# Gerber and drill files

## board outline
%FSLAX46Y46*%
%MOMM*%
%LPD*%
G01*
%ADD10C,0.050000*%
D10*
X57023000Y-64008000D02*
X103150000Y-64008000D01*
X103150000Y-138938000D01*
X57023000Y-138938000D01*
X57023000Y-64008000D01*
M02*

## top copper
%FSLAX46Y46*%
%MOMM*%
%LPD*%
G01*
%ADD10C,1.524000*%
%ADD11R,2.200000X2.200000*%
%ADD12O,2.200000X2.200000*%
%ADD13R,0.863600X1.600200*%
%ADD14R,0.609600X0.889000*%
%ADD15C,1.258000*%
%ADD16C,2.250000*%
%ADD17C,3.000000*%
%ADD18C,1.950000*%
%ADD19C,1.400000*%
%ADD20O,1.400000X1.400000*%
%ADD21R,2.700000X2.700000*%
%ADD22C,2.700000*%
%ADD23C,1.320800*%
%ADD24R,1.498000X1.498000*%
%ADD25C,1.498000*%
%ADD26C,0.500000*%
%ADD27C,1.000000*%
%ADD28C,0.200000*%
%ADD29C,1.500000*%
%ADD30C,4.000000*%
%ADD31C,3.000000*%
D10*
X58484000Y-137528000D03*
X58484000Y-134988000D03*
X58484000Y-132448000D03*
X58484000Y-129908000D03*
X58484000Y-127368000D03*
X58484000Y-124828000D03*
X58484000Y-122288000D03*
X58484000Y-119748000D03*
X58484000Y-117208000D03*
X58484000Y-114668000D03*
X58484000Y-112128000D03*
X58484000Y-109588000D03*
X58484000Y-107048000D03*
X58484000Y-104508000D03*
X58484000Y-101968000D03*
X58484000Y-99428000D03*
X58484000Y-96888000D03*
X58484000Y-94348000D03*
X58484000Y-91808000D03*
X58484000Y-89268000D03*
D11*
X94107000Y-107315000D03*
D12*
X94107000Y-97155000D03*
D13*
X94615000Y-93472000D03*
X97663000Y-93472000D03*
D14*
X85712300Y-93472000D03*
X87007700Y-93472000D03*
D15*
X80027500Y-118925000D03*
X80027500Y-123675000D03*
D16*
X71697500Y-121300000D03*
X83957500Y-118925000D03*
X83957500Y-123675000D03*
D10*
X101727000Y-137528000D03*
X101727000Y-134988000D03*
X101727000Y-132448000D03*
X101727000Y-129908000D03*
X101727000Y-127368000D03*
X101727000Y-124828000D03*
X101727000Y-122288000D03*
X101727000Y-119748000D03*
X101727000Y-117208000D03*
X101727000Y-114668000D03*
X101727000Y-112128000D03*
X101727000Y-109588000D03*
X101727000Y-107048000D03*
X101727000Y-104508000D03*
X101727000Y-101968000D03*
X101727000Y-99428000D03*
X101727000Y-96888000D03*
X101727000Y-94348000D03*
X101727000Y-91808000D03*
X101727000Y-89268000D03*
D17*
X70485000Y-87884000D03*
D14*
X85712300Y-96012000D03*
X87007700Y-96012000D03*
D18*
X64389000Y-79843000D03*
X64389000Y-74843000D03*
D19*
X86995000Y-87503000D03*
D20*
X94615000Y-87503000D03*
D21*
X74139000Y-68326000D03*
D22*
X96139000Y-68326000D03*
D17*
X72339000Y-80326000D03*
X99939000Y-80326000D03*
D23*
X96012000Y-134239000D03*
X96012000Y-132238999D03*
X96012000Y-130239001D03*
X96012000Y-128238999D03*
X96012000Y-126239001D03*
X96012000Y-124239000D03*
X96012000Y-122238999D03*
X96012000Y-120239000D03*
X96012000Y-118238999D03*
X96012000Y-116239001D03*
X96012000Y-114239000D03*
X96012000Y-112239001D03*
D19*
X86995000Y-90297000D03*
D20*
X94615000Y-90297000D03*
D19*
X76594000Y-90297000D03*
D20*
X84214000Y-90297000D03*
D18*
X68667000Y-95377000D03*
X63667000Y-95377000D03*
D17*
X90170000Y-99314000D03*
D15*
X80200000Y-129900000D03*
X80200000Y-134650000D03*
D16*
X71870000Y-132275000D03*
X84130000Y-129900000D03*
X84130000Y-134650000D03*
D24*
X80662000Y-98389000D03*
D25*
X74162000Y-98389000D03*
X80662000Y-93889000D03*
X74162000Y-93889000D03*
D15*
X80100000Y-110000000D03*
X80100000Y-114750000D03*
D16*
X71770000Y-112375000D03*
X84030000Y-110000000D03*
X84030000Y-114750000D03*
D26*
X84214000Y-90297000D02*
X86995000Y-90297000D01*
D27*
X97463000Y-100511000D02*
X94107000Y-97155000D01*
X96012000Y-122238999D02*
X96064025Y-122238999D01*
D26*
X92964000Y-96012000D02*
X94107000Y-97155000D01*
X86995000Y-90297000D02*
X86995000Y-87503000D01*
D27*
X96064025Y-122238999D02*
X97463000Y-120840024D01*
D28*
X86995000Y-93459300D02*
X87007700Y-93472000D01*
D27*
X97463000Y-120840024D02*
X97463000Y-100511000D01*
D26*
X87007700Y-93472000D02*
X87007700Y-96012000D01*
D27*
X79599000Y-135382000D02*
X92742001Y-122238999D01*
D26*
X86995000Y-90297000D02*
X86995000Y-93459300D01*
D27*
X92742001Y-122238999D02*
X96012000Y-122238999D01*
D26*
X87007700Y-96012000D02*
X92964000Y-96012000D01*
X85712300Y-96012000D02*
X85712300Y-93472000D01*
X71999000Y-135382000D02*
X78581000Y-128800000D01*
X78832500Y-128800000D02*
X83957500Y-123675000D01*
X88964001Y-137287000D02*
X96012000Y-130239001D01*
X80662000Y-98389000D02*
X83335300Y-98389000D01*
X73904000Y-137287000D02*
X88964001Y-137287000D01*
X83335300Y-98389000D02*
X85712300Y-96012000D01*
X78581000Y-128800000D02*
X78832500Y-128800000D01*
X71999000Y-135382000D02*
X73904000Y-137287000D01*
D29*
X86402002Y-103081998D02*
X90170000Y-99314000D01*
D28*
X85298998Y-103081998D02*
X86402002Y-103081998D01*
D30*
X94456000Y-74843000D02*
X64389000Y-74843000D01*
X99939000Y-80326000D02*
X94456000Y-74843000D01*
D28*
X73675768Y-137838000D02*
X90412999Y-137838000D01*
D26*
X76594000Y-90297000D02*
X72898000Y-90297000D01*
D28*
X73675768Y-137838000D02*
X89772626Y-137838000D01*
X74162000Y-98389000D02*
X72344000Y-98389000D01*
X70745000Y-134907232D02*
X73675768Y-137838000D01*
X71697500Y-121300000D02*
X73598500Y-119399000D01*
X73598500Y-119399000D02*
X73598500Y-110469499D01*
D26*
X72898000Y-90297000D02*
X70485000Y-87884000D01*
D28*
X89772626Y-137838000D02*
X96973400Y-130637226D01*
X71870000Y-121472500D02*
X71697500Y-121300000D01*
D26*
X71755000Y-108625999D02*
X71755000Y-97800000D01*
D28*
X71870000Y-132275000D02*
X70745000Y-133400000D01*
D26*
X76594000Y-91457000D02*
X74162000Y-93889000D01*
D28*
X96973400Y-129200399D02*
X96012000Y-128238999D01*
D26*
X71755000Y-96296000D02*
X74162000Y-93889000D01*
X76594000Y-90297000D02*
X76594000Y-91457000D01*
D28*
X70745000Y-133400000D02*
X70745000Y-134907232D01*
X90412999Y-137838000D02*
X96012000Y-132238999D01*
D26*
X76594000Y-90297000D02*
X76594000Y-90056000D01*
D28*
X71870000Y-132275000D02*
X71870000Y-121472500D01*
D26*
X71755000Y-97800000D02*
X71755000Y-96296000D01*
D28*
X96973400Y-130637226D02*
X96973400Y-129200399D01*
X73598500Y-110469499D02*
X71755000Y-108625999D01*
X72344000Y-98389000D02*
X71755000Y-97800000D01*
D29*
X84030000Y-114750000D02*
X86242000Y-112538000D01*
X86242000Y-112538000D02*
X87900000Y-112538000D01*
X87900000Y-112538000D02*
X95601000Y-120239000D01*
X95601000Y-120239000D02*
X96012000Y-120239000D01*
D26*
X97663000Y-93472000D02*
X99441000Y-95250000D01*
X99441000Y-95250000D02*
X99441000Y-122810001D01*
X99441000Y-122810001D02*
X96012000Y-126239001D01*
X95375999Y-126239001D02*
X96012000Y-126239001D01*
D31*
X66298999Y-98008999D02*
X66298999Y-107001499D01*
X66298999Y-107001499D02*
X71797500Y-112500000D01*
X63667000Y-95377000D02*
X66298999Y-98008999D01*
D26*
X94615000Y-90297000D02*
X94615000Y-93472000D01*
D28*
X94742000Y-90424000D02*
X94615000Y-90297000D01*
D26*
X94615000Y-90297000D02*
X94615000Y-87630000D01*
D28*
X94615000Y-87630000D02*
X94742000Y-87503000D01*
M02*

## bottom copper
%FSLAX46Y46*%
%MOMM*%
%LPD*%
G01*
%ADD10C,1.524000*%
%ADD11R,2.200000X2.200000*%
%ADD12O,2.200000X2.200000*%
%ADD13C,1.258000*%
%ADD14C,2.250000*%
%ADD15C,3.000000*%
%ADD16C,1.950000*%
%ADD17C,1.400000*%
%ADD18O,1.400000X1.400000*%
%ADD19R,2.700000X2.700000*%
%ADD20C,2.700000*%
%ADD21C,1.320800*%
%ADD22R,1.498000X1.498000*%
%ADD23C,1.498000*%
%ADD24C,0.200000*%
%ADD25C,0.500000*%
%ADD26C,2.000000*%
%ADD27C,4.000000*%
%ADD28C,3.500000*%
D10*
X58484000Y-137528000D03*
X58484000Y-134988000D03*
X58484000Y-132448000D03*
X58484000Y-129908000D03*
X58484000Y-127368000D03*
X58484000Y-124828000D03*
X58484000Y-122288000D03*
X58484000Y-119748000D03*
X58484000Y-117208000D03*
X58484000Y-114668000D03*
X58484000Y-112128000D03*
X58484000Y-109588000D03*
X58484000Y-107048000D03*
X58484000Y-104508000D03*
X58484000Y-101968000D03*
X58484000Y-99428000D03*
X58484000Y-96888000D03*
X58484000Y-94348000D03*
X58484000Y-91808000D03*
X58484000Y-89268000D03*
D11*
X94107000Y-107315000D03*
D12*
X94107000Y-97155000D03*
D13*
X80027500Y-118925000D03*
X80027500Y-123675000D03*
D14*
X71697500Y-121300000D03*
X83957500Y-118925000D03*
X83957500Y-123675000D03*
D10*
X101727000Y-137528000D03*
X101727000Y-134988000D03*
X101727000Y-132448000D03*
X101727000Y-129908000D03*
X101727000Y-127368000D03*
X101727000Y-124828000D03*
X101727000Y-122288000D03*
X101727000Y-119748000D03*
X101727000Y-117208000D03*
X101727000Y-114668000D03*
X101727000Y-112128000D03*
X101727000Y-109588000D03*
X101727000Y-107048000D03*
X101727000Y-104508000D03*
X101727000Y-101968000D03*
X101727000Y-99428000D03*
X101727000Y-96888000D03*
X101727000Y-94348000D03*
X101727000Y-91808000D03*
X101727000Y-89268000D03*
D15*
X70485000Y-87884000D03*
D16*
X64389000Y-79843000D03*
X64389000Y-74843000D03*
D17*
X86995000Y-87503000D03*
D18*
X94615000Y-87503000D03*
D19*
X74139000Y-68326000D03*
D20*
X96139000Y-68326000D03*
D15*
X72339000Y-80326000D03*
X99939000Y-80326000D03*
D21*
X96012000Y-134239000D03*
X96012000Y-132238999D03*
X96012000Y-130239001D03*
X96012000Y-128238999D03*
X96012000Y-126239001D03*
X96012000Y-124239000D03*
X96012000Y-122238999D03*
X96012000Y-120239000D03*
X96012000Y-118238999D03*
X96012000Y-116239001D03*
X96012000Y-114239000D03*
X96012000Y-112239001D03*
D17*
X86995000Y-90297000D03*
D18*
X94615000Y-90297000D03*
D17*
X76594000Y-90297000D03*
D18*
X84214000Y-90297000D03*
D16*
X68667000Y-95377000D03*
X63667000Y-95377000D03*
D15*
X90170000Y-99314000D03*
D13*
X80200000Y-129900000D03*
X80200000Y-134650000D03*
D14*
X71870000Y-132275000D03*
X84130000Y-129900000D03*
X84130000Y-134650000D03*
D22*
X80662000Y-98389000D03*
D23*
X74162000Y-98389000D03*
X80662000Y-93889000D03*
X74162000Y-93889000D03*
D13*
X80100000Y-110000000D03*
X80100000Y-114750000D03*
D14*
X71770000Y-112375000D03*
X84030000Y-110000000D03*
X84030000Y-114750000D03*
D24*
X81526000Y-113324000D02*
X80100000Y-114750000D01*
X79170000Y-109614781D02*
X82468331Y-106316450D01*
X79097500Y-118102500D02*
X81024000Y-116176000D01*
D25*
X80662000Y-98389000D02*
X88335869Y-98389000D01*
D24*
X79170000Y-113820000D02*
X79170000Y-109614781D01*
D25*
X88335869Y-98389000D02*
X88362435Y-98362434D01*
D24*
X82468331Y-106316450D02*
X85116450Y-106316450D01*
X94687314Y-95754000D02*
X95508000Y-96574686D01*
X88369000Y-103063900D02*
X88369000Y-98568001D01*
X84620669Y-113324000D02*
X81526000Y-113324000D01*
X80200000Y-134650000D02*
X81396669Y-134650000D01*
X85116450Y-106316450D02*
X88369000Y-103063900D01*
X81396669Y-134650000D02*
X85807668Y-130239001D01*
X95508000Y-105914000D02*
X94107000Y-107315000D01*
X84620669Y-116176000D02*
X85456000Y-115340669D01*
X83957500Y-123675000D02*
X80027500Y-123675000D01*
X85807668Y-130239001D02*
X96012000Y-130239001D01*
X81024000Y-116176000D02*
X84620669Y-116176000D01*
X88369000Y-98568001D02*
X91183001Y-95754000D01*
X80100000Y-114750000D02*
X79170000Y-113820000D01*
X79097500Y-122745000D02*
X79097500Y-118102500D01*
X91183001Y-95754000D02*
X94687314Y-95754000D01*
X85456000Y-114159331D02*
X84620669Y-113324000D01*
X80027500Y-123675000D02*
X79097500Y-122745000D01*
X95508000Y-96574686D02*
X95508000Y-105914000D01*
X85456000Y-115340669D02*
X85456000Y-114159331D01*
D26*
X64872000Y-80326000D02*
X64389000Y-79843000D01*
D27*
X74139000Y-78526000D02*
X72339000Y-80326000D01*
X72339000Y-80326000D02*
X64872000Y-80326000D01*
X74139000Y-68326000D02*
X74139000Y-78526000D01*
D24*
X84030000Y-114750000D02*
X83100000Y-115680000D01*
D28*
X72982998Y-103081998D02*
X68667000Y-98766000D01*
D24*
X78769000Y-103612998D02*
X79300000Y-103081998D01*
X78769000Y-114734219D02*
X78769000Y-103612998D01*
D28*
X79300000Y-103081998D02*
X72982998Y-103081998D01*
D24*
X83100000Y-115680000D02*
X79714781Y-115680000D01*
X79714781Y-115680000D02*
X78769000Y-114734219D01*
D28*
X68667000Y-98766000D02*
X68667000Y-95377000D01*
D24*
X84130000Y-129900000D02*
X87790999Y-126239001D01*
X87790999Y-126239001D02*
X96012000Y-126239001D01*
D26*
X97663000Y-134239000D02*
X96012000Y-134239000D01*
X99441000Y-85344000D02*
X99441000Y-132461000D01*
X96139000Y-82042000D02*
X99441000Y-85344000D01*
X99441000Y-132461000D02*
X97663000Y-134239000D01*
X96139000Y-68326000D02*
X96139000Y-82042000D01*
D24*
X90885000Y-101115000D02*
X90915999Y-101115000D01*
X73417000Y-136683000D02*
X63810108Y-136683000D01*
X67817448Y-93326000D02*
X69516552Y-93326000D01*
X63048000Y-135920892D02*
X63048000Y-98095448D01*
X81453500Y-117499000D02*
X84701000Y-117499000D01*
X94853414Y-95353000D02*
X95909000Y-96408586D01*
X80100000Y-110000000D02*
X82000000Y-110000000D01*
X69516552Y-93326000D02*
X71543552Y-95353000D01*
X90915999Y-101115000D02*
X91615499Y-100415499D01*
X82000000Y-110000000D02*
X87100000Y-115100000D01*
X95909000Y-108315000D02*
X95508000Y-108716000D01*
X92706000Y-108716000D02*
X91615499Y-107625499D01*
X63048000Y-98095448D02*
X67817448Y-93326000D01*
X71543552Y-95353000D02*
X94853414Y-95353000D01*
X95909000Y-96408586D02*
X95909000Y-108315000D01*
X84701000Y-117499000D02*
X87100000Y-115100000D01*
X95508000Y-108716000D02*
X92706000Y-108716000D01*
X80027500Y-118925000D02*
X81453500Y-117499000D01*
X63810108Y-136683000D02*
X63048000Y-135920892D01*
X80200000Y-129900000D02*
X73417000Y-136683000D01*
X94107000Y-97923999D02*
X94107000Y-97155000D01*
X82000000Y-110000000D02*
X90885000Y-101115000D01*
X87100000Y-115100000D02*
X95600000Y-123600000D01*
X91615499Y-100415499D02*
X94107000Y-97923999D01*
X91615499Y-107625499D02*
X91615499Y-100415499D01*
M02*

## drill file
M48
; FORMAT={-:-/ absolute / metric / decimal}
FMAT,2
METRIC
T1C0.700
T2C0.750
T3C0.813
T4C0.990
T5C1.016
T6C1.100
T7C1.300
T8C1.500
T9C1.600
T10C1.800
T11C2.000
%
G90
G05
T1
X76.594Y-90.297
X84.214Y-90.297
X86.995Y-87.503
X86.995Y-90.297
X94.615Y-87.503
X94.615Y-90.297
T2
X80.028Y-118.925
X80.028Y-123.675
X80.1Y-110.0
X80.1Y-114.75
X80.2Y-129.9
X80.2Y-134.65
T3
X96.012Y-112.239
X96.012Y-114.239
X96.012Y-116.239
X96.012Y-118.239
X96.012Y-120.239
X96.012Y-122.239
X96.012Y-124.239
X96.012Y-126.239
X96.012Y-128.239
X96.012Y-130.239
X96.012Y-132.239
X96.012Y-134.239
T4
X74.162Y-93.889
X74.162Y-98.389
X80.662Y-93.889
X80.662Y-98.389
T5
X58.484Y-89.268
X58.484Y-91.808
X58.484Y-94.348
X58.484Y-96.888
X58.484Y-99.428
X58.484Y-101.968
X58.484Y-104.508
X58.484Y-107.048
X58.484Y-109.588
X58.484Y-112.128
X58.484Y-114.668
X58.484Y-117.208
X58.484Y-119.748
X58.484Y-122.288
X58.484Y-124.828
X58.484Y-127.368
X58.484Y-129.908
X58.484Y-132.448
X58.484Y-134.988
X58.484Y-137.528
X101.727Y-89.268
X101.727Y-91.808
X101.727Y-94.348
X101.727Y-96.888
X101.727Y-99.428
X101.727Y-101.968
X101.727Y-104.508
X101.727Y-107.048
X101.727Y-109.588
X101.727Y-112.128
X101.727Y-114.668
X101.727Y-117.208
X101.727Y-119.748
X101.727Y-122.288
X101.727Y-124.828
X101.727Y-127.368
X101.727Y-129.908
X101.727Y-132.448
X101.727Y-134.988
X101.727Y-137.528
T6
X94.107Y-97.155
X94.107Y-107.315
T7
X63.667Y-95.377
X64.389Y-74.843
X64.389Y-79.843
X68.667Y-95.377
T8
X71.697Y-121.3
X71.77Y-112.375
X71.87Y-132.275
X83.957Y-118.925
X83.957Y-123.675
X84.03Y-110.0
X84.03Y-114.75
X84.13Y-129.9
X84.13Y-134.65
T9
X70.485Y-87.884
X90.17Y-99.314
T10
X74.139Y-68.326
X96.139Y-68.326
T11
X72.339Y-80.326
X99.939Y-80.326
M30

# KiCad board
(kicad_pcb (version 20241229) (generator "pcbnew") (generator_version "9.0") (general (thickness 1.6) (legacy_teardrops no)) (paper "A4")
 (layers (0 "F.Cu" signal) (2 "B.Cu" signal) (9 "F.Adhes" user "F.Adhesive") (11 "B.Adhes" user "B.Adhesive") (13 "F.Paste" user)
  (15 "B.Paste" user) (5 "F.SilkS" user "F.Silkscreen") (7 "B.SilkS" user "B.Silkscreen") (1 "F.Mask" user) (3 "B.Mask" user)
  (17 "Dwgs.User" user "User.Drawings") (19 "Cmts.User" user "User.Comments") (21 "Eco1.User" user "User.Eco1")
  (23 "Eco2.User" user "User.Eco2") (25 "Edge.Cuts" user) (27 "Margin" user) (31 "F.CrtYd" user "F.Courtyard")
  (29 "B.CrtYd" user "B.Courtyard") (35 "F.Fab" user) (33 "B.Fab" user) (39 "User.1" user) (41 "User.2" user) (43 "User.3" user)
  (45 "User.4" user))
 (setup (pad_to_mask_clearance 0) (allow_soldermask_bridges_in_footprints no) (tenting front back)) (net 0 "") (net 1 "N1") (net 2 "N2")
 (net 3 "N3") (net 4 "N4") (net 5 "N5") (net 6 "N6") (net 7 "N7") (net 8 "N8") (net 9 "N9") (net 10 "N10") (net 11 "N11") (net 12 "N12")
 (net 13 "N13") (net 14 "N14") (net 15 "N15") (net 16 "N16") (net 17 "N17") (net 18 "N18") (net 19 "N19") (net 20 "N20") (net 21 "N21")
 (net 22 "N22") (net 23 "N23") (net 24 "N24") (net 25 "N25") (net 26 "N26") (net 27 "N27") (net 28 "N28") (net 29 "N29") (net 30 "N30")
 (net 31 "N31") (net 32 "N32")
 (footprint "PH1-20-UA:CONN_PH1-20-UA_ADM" (layer "F.Cu") (at 58.484 137.528 90)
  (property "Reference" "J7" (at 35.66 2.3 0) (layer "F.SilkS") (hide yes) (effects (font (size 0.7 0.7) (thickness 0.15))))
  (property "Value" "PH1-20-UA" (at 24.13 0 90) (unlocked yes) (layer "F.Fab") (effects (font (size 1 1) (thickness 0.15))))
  (pad "1" thru_hole circle (at 0 0 90) (size 1.524 1.524) (drill 1.016) (layers "*.Cu" "*.Mask") (remove_unused_layers no))
  (pad "2" thru_hole circle (at 2.54 0 90) (size 1.524 1.524) (drill 1.016) (layers "*.Cu" "*.Mask") (remove_unused_layers no))
  (pad "3" thru_hole circle (at 5.08 0 90) (size 1.524 1.524) (drill 1.016) (layers "*.Cu" "*.Mask") (remove_unused_layers no))
  (pad "4" thru_hole circle (at 7.62 0 90) (size 1.524 1.524) (drill 1.016) (layers "*.Cu" "*.Mask") (remove_unused_layers no))
  (pad "5" thru_hole circle (at 10.16 0 90) (size 1.524 1.524) (drill 1.016) (layers "*.Cu" "*.Mask") (remove_unused_layers no))
  (pad "6" thru_hole circle (at 12.7 0 90) (size 1.524 1.524) (drill 1.016) (layers "*.Cu" "*.Mask") (remove_unused_layers no))
  (pad "7" thru_hole circle (at 15.24 0 90) (size 1.524 1.524) (drill 1.016) (layers "*.Cu" "*.Mask") (remove_unused_layers no) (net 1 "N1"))
  (pad "8" thru_hole circle (at 17.78 0 90) (size 1.524 1.524) (drill 1.016) (layers "*.Cu" "*.Mask") (remove_unused_layers no) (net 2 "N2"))
  (pad "9" thru_hole circle (at 20.32 0 90) (size 1.524 1.524) (drill 1.016) (layers "*.Cu" "*.Mask") (remove_unused_layers no) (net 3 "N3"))
  (pad "10" thru_hole circle (at 22.86 0 90) (size 1.524 1.524) (drill 1.016) (layers "*.Cu" "*.Mask") (remove_unused_layers no)
   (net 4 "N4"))
  (pad "11" thru_hole circle (at 25.4 0 90) (size 1.524 1.524) (drill 1.016) (layers "*.Cu" "*.Mask") (remove_unused_layers no) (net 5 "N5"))
  (pad "12" thru_hole circle (at 27.94 0 90) (size 1.524 1.524) (drill 1.016) (layers "*.Cu" "*.Mask") (remove_unused_layers no)
   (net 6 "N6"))
  (pad "13" thru_hole circle (at 30.48 0 90) (size 1.524 1.524) (drill 1.016) (layers "*.Cu" "*.Mask") (remove_unused_layers no)
   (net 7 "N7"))
  (pad "14" thru_hole circle (at 33.02 0 90) (size 1.524 1.524) (drill 1.016) (layers "*.Cu" "*.Mask") (remove_unused_layers no)
   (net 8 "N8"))
  (pad "15" thru_hole circle (at 35.56 0 90) (size 1.524 1.524) (drill 1.016) (layers "*.Cu" "*.Mask") (remove_unused_layers no)
   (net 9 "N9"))
  (pad "16" thru_hole circle (at 38.1 0 90) (size 1.524 1.524) (drill 1.016) (layers "*.Cu" "*.Mask") (remove_unused_layers no)
   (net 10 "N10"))
  (pad "17" thru_hole circle (at 40.64 0 90) (size 1.524 1.524) (drill 1.016) (layers "*.Cu" "*.Mask") (remove_unused_layers no)
   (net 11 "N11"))
  (pad "18" thru_hole circle (at 43.18 0 90) (size 1.524 1.524) (drill 1.016) (layers "*.Cu" "*.Mask") (remove_unused_layers no)
   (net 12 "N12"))
  (pad "19" thru_hole circle (at 45.72 0 90) (size 1.524 1.524) (drill 1.016) (layers "*.Cu" "*.Mask") (remove_unused_layers no)
   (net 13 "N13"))
  (pad "20" thru_hole circle (at 48.26 0 90) (size 1.524 1.524) (drill 1.016) (layers "*.Cu" "*.Mask") (remove_unused_layers no)
   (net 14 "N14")))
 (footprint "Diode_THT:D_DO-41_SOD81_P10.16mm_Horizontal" (layer "F.Cu") (at 94.107 107.315 90)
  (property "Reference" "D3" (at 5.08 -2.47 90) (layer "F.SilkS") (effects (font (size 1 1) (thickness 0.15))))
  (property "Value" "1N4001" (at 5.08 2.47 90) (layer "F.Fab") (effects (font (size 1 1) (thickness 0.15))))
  (pad "1" thru_hole rect (at 0 0 90) (size 2.2 2.2) (drill 1.1) (layers "*.Cu" "*.Mask") (remove_unused_layers no) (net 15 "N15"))
  (pad "2" thru_hole oval (at 10.16 0 90) (size 2.2 2.2) (drill 1.1) (layers "*.Cu" "*.Mask") (remove_unused_layers no) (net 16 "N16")))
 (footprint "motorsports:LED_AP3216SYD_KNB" (layer "F.Cu") (at 96.139 93.472)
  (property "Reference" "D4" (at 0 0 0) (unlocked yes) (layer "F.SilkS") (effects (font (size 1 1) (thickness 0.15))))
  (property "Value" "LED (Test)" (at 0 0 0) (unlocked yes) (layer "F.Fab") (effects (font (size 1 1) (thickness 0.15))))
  (pad "1" smd rect (at -1.524 0) (size 0.8636 1.6002) (layers "F.Cu" "F.Mask" "F.Paste") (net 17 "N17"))
  (pad "2" smd rect (at 1.524 0) (size 0.8636 1.6002) (layers "F.Cu" "F.Mask" "F.Paste") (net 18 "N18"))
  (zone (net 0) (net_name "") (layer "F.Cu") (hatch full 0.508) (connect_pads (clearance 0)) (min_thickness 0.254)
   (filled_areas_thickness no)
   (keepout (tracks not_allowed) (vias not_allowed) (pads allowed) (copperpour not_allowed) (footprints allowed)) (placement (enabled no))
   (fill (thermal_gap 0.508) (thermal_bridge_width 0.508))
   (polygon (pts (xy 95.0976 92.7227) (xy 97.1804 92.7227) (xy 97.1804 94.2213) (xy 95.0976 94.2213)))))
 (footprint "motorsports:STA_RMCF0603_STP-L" (layer "F.Cu") (at 86.36 93.472)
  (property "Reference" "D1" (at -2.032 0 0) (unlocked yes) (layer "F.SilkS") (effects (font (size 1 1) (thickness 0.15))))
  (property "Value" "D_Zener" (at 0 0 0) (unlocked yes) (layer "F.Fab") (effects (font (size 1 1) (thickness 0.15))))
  (pad "1" smd rect (at -0.6477 0) (size 0.6096 0.889) (layers "F.Cu" "F.Mask" "F.Paste") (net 15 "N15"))
  (pad "2" smd rect (at 0.6477 0) (size 0.6096 0.889) (layers "F.Cu" "F.Mask" "F.Paste") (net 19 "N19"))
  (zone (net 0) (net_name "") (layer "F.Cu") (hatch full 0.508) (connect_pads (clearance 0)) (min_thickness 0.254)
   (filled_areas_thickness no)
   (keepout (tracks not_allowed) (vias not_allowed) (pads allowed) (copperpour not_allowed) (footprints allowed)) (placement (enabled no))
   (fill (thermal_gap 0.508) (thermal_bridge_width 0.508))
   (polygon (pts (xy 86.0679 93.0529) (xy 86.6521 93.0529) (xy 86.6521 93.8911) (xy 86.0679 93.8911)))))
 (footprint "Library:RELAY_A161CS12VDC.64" (layer "F.Cu") (at 77.9475 121.3)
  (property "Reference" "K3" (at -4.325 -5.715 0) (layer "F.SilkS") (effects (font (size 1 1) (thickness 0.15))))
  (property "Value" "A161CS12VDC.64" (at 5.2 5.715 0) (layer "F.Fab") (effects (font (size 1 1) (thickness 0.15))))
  (pad "A1" thru_hole circle (at 2.08 -2.375) (size 1.258 1.258) (drill 0.75) (layers "*.Cu" "*.Mask") (remove_unused_layers no)
   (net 16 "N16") (solder_mask_margin 0.102))
  (pad "A2" thru_hole circle (at 2.08 2.375) (size 1.258 1.258) (drill 0.75) (layers "*.Cu" "*.Mask") (remove_unused_layers no)
   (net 15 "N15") (solder_mask_margin 0.102))
  (pad "COM" thru_hole circle (at -6.25 0) (size 2.25 2.25) (drill 1.5) (layers "*.Cu" "*.Mask") (remove_unused_layers no) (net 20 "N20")
   (solder_mask_margin 0.102))
  (pad "NC" thru_hole circle (at 6.01 -2.375) (size 2.25 2.25) (drill 1.5) (layers "*.Cu" "*.Mask") (remove_unused_layers no) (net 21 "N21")
   (solder_mask_margin 0.102))
  (pad "NO" thru_hole circle (at 6.01 2.375) (size 2.25 2.25) (drill 1.5) (layers "*.Cu" "*.Mask") (remove_unused_layers no) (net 15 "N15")
   (solder_mask_margin 0.102)))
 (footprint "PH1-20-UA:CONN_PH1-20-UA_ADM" (layer "F.Cu") (at 101.727 137.528 90)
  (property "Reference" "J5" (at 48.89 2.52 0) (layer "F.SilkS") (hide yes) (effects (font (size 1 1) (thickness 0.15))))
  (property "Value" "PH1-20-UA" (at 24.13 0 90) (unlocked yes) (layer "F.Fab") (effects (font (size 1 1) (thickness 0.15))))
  (pad "1" thru_hole circle (at 0 0 90) (size 1.524 1.524) (drill 1.016) (layers "*.Cu" "*.Mask") (remove_unused_layers no))
  (pad "2" thru_hole circle (at 2.54 0 90) (size 1.524 1.524) (drill 1.016) (layers "*.Cu" "*.Mask") (remove_unused_layers no))
  (pad "3" thru_hole circle (at 5.08 0 90) (size 1.524 1.524) (drill 1.016) (layers "*.Cu" "*.Mask") (remove_unused_layers no))
  (pad "4" thru_hole circle (at 7.62 0 90) (size 1.524 1.524) (drill 1.016) (layers "*.Cu" "*.Mask") (remove_unused_layers no))
  (pad "5" thru_hole circle (at 10.16 0 90) (size 1.524 1.524) (drill 1.016) (layers "*.Cu" "*.Mask") (remove_unused_layers no))
  (pad "6" thru_hole circle (at 12.7 0 90) (size 1.524 1.524) (drill 1.016) (layers "*.Cu" "*.Mask") (remove_unused_layers no))
  (pad "7" thru_hole circle (at 15.24 0 90) (size 1.524 1.524) (drill 1.016) (layers "*.Cu" "*.Mask") (remove_unused_layers no))
  (pad "8" thru_hole circle (at 17.78 0 90) (size 1.524 1.524) (drill 1.016) (layers "*.Cu" "*.Mask") (remove_unused_layers no))
  (pad "9" thru_hole circle (at 20.32 0 90) (size 1.524 1.524) (drill 1.016) (layers "*.Cu" "*.Mask") (remove_unused_layers no))
  (pad "10" thru_hole circle (at 22.86 0 90) (size 1.524 1.524) (drill 1.016) (layers "*.Cu" "*.Mask") (remove_unused_layers no))
  (pad "11" thru_hole circle (at 25.4 0 90) (size 1.524 1.524) (drill 1.016) (layers "*.Cu" "*.Mask") (remove_unused_layers no))
  (pad "12" thru_hole circle (at 27.94 0 90) (size 1.524 1.524) (drill 1.016) (layers "*.Cu" "*.Mask") (remove_unused_layers no))
  (pad "13" thru_hole circle (at 30.48 0 90) (size 1.524 1.524) (drill 1.016) (layers "*.Cu" "*.Mask") (remove_unused_layers no))
  (pad "14" thru_hole circle (at 33.02 0 90) (size 1.524 1.524) (drill 1.016) (layers "*.Cu" "*.Mask") (remove_unused_layers no))
  (pad "15" thru_hole circle (at 35.56 0 90) (size 1.524 1.524) (drill 1.016) (layers "*.Cu" "*.Mask") (remove_unused_layers no))
  (pad "16" thru_hole circle (at 38.1 0 90) (size 1.524 1.524) (drill 1.016) (layers "*.Cu" "*.Mask") (remove_unused_layers no))
  (pad "17" thru_hole circle (at 40.64 0 90) (size 1.524 1.524) (drill 1.016) (layers "*.Cu" "*.Mask") (remove_unused_layers no))
  (pad "18" thru_hole circle (at 43.18 0 90) (size 1.524 1.524) (drill 1.016) (layers "*.Cu" "*.Mask") (remove_unused_layers no))
  (pad "19" thru_hole circle (at 45.72 0 90) (size 1.524 1.524) (drill 1.016) (layers "*.Cu" "*.Mask") (remove_unused_layers no))
  (pad "20" thru_hole circle (at 48.26 0 90) (size 1.524 1.524) (drill 1.016) (layers "*.Cu" "*.Mask") (remove_unused_layers no)))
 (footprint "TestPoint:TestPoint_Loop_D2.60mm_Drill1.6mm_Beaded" (layer "F.Cu") (at 70.485 87.884)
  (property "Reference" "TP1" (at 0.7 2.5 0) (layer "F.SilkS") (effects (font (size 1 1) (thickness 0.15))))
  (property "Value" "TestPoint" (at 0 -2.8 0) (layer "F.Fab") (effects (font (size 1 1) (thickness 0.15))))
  (pad "1" thru_hole circle (at 0 0) (size 3 3) (drill 1.6) (layers "*.Cu" "*.Mask") (remove_unused_layers no) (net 20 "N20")))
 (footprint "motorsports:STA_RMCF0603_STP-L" (layer "F.Cu") (at 86.36 96.012)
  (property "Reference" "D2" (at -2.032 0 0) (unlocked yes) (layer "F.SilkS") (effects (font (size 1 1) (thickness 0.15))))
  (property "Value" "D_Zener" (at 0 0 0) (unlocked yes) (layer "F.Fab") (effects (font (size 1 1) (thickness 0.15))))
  (pad "1" smd rect (at -0.6477 0) (size 0.6096 0.889) (layers "F.Cu" "F.Mask" "F.Paste") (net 15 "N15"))
  (pad "2" smd rect (at 0.6477 0) (size 0.6096 0.889) (layers "F.Cu" "F.Mask" "F.Paste") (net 19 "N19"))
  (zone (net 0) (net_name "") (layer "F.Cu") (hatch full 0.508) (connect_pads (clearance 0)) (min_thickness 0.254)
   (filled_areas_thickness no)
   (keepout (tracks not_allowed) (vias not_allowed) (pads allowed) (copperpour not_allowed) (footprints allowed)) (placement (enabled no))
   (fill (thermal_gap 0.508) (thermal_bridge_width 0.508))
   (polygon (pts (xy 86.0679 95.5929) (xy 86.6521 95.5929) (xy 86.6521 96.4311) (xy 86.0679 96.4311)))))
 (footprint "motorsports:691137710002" (layer "F.Cu") (at 64.389 77.343 90)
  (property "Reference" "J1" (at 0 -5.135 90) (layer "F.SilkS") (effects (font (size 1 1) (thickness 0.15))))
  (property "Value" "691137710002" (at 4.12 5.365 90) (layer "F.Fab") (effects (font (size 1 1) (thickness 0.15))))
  (pad "1" thru_hole circle (at -2.5 0 90) (size 1.95 1.95) (drill 1.3) (layers "*.Cu" "*.Mask") (remove_unused_layers no) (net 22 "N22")
   (solder_mask_margin 0.102))
  (pad "2" thru_hole circle (at 2.5 0 90) (size 1.95 1.95) (drill 1.3) (layers "*.Cu" "*.Mask") (remove_unused_layers no) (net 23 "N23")
   (solder_mask_margin 0.102)))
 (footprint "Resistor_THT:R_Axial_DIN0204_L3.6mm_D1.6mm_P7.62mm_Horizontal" (layer "F.Cu") (at 86.995 87.503)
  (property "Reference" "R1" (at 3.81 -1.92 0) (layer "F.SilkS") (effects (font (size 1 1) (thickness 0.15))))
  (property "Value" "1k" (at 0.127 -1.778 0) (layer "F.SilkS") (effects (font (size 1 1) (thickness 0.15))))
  (pad "1" thru_hole circle (at 0 0) (size 1.4 1.4) (drill 0.7) (layers "*.Cu" "*.Mask") (remove_unused_layers no) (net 19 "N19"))
  (pad "2" thru_hole oval (at 7.62 0) (size 1.4 1.4) (drill 0.7) (layers "*.Cu" "*.Mask") (remove_unused_layers no) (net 17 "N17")))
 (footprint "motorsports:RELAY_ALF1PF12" (layer "F.Cu") (at 86.139 74.326)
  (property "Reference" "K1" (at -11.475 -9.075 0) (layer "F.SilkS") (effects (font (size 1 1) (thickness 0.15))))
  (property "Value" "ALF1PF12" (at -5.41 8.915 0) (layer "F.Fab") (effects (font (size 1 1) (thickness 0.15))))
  (pad "1" thru_hole rect (at -12 -6) (size 2.7 2.7) (drill 1.8) (layers "*.Cu" "*.Mask") (remove_unused_layers no) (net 22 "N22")
   (solder_mask_margin 0.102))
  (pad "2" thru_hole circle (at 10 -6) (size 2.7 2.7) (drill 1.8) (layers "*.Cu" "*.Mask") (remove_unused_layers no) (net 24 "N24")
   (solder_mask_margin 0.102))
  (pad "3" thru_hole circle (at -13.8 6) (size 3 3) (drill 2) (layers "*.Cu" "*.Mask") (remove_unused_layers no) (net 22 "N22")
   (solder_mask_margin 0.102))
  (pad "4" thru_hole circle (at 13.8 6) (size 3 3) (drill 2) (layers "*.Cu" "*.Mask") (remove_unused_layers no) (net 23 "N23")
   (solder_mask_margin 0.102)))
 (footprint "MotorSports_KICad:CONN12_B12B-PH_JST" (layer "F.Cu") (at 96.012 134.239 90)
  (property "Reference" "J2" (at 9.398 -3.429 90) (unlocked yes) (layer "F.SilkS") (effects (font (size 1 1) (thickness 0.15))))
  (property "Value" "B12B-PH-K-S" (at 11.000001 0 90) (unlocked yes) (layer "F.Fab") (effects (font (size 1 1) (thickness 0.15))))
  (pad "1" thru_hole circle (at 0 0 90) (size 1.3208 1.3208) (drill 0.8128) (layers "*.Cu" "*.Mask") (remove_unused_layers no)
   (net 24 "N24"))
  (pad "2" thru_hole circle (at 2.000001 0 90) (size 1.3208 1.3208) (drill 0.8128) (layers "*.Cu" "*.Mask") (remove_unused_layers no)
   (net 20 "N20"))
  (pad "3" thru_hole circle (at 3.999999 0 90) (size 1.3208 1.3208) (drill 0.8128) (layers "*.Cu" "*.Mask") (remove_unused_layers no)
   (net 15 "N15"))
  (pad "4" thru_hole circle (at 6.000001 0 90) (size 1.3208 1.3208) (drill 0.8128) (layers "*.Cu" "*.Mask") (remove_unused_layers no)
   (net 20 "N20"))
  (pad "5" thru_hole circle (at 7.999999 0 90) (size 1.3208 1.3208) (drill 0.8128) (layers "*.Cu" "*.Mask") (remove_unused_layers no)
   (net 18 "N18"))
  (pad "6" thru_hole circle (at 10 0 90) (size 1.3208 1.3208) (drill 0.8128) (layers "*.Cu" "*.Mask") (remove_unused_layers no)
   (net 16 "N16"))
  (pad "7" thru_hole circle (at 12.000001 0 90) (size 1.3208 1.3208) (drill 0.8128) (layers "*.Cu" "*.Mask") (remove_unused_layers no)
   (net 19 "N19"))
  (pad "8" thru_hole circle (at 14 0 90) (size 1.3208 1.3208) (drill 0.8128) (layers "*.Cu" "*.Mask") (remove_unused_layers no)
   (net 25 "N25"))
  (pad "9" thru_hole circle (at 16.000001 0 90) (size 1.3208 1.3208) (drill 0.8128) (layers "*.Cu" "*.Mask") (remove_unused_layers no)
   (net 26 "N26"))
  (pad "10" thru_hole circle (at 17.999999 0 90) (size 1.3208 1.3208) (drill 0.8128) (layers "*.Cu" "*.Mask") (remove_unused_layers no)
   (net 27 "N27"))
  (pad "11" thru_hole circle (at 20 0 90) (size 1.3208 1.3208) (drill 0.8128) (layers "*.Cu" "*.Mask") (remove_unused_layers no)
   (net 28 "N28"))
  (pad "12" thru_hole circle (at 21.999999 0 90) (size 1.3208 1.3208) (drill 0.8128) (layers "*.Cu" "*.Mask") (remove_unused_layers no)
   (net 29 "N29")))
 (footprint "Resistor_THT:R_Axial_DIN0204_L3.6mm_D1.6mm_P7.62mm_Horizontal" (layer "F.Cu") (at 86.995 90.297)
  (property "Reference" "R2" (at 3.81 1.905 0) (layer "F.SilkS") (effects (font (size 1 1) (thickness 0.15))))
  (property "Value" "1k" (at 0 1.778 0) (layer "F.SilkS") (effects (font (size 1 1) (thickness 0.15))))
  (pad "1" thru_hole circle (at 0 0) (size 1.4 1.4) (drill 0.7) (layers "*.Cu" "*.Mask") (remove_unused_layers no) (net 19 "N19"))
  (pad "2" thru_hole oval (at 7.62 0) (size 1.4 1.4) (drill 0.7) (layers "*.Cu" "*.Mask") (remove_unused_layers no) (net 17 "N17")))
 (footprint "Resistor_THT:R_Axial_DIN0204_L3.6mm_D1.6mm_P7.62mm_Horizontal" (layer "F.Cu") (at 76.594 90.297)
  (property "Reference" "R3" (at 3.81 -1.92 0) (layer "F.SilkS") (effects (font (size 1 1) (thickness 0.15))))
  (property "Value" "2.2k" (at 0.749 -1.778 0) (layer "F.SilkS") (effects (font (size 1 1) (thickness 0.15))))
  (pad "1" thru_hole circle (at 0 0) (size 1.4 1.4) (drill 0.7) (layers "*.Cu" "*.Mask") (remove_unused_layers no) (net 20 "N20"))
  (pad "2" thru_hole oval (at 7.62 0) (size 1.4 1.4) (drill 0.7) (layers "*.Cu" "*.Mask") (remove_unused_layers no) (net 19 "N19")))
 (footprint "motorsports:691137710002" (layer "F.Cu") (at 66.167 95.377 180)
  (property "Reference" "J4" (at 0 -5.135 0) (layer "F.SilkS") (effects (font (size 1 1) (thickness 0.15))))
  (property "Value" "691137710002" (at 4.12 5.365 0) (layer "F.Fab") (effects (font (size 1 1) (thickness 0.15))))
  (pad "1" thru_hole circle (at -2.5 0 180) (size 1.95 1.95) (drill 1.3) (layers "*.Cu" "*.Mask") (remove_unused_layers no) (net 25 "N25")
   (solder_mask_margin 0.102))
  (pad "2" thru_hole circle (at 2.5 0 180) (size 1.95 1.95) (drill 1.3) (layers "*.Cu" "*.Mask") (remove_unused_layers no) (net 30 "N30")
   (solder_mask_margin 0.102)))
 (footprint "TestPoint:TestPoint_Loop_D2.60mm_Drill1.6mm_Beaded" (layer "F.Cu") (at 90.17 99.314)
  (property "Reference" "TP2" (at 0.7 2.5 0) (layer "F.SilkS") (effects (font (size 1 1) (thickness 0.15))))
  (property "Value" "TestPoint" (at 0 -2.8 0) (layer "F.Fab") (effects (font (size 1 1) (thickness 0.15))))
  (pad "1" thru_hole circle (at 0 0) (size 3 3) (drill 1.6) (layers "*.Cu" "*.Mask") (remove_unused_layers no) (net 19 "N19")))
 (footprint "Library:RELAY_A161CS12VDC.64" (layer "F.Cu") (at 78.12 132.275)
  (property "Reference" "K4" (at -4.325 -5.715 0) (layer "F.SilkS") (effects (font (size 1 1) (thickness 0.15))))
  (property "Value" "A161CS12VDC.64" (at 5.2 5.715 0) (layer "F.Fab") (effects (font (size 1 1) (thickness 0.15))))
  (pad "A1" thru_hole circle (at 2.08 -2.375) (size 1.258 1.258) (drill 0.75) (layers "*.Cu" "*.Mask") (remove_unused_layers no)
   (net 16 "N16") (solder_mask_margin 0.102))
  (pad "A2" thru_hole circle (at 2.08 2.375) (size 1.258 1.258) (drill 0.75) (layers "*.Cu" "*.Mask") (remove_unused_layers no)
   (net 15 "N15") (solder_mask_margin 0.102))
  (pad "COM" thru_hole circle (at -6.25 0) (size 2.25 2.25) (drill 1.5) (layers "*.Cu" "*.Mask") (remove_unused_layers no) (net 20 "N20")
   (solder_mask_margin 0.102))
  (pad "NC" thru_hole circle (at 6.01 -2.375) (size 2.25 2.25) (drill 1.5) (layers "*.Cu" "*.Mask") (remove_unused_layers no) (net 18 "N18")
   (solder_mask_margin 0.102))
  (pad "NO" thru_hole circle (at 6.01 2.375) (size 2.25 2.25) (drill 1.5) (layers "*.Cu" "*.Mask") (remove_unused_layers no) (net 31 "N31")
   (solder_mask_margin 0.102)))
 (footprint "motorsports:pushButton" (layer "F.Cu") (at 77.412 96.139 180)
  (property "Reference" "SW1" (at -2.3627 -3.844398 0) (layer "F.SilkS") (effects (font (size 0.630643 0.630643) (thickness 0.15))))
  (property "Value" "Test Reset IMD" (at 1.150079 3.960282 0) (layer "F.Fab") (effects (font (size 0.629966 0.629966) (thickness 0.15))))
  (pad "1" thru_hole rect (at -3.25 -2.25 180) (size 1.498 1.498) (drill 0.99) (layers "*.Cu" "*.Mask") (remove_unused_layers no)
   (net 15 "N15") (solder_mask_margin 0.102))
  (pad "2" thru_hole circle (at 3.25 -2.25 180) (size 1.498 1.498) (drill 0.99) (layers "*.Cu" "*.Mask") (remove_unused_layers no)
   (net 20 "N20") (solder_mask_margin 0.102))
  (pad "3" thru_hole circle (at -3.25 2.25 180) (size 1.498 1.498) (drill 0.99) (layers "*.Cu" "*.Mask") (remove_unused_layers no)
   (solder_mask_margin 0.102))
  (pad "4" thru_hole circle (at 3.25 2.25 180) (size 1.498 1.498) (drill 0.99) (layers "*.Cu" "*.Mask") (remove_unused_layers no)
   (solder_mask_margin 0.102)))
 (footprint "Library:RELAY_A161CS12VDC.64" (layer "F.Cu") (at 78.02 112.375)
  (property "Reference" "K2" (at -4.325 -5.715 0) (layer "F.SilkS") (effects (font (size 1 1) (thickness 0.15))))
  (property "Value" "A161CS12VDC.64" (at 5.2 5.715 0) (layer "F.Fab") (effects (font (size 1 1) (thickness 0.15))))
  (pad "A1" thru_hole circle (at 2.08 -2.375) (size 1.258 1.258) (drill 0.75) (layers "*.Cu" "*.Mask") (remove_unused_layers no)
   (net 16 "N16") (solder_mask_margin 0.102))
  (pad "A2" thru_hole circle (at 2.08 2.375) (size 1.258 1.258) (drill 0.75) (layers "*.Cu" "*.Mask") (remove_unused_layers no)
   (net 15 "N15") (solder_mask_margin 0.102))
  (pad "COM" thru_hole circle (at -6.25 0) (size 2.25 2.25) (drill 1.5) (layers "*.Cu" "*.Mask") (remove_unused_layers no) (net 30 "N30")
   (solder_mask_margin 0.102))
  (pad "NC" thru_hole circle (at 6.01 -2.375) (size 2.25 2.25) (drill 1.5) (layers "*.Cu" "*.Mask") (remove_unused_layers no) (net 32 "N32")
   (solder_mask_margin 0.102))
  (pad "NO" thru_hole circle (at 6.01 2.375) (size 2.25 2.25) (drill 1.5) (layers "*.Cu" "*.Mask") (remove_unused_layers no) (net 25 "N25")
   (solder_mask_margin 0.102)))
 (gr_rect (start 57.023 64.008) (end 103.15 138.938) (stroke (width 0.05) (type default)) (fill no) (layer "Edge.Cuts"))
 (segment (start 84.214 90.297) (end 86.995 90.297) (width 0.5) (layer "F.Cu") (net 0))
 (segment (start 97.463 100.511) (end 94.107 97.155) (width 1) (layer "F.Cu") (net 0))
 (segment (start 96.012 122.238999) (end 96.064025 122.238999) (width 1) (layer "F.Cu") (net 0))
 (segment (start 92.964 96.012) (end 94.107 97.155) (width 0.5) (layer "F.Cu") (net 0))
 (segment (start 86.995 90.297) (end 86.995 87.503) (width 0.5) (layer "F.Cu") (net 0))
 (segment (start 96.064025 122.238999) (end 97.463 120.840024) (width 1) (layer "F.Cu") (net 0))
 (segment (start 86.995 93.4593) (end 87.0077 93.472) (width 0.2) (layer "F.Cu") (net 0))
 (segment (start 97.463 120.840024) (end 97.463 100.511) (width 1) (layer "F.Cu") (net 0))
 (segment (start 87.0077 93.472) (end 87.0077 96.012) (width 0.5) (layer "F.Cu") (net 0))
 (segment (start 79.599 135.382) (end 92.742001 122.238999) (width 1) (layer "F.Cu") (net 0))
 (segment (start 86.995 90.297) (end 86.995 93.4593) (width 0.5) (layer "F.Cu") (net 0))
 (segment (start 92.742001 122.238999) (end 96.012 122.238999) (width 1) (layer "F.Cu") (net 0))
 (segment (start 87.0077 96.012) (end 92.964 96.012) (width 0.5) (layer "F.Cu") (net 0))
 (segment (start 85.7123 96.012) (end 85.7123 93.472) (width 0.5) (layer "F.Cu") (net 15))
 (segment (start 71.999 135.382) (end 78.581 128.8) (width 0.5) (layer "F.Cu") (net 15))
 (segment (start 78.8325 128.8) (end 83.9575 123.675) (width 0.5) (layer "F.Cu") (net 15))
 (segment (start 88.964001 137.287) (end 96.012 130.239001) (width 0.5) (layer "F.Cu") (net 15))
 (segment (start 80.662 98.389) (end 83.3353 98.389) (width 0.5) (layer "F.Cu") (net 15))
 (segment (start 73.904 137.287) (end 88.964001 137.287) (width 0.5) (layer "F.Cu") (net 15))
 (segment (start 83.3353 98.389) (end 85.7123 96.012) (width 0.5) (layer "F.Cu") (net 15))
 (segment (start 78.581 128.8) (end 78.8325 128.8) (width 0.5) (layer "F.Cu") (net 15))
 (segment (start 71.999 135.382) (end 73.904 137.287) (width 0.5) (layer "F.Cu") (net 15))
 (segment (start 81.526 113.324) (end 80.1 114.75) (width 0.2) (layer "B.Cu") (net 15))
 (segment (start 79.17 109.614781) (end 82.468331 106.31645) (width 0.2) (layer "B.Cu") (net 15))
 (segment (start 79.0975 118.1025) (end 81.024 116.176) (width 0.2) (layer "B.Cu") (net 15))
 (segment (start 80.662 98.389) (end 88.335869 98.389) (width 0.5) (layer "B.Cu") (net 15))
 (segment (start 79.17 113.82) (end 79.17 109.614781) (width 0.2) (layer "B.Cu") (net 15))
 (segment (start 88.335869 98.389) (end 88.362435 98.362434) (width 0.5) (layer "B.Cu") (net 15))
 (segment (start 82.468331 106.31645) (end 85.11645 106.31645) (width 0.2) (layer "B.Cu") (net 15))
 (segment (start 94.687314 95.754) (end 95.508 96.574686) (width 0.2) (layer "B.Cu") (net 15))
 (segment (start 88.369 103.0639) (end 88.369 98.568001) (width 0.2) (layer "B.Cu") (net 15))
 (segment (start 84.620669 113.324) (end 81.526 113.324) (width 0.2) (layer "B.Cu") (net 15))
 (segment (start 80.2 134.65) (end 81.396669 134.65) (width 0.2) (layer "B.Cu") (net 15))
 (segment (start 85.11645 106.31645) (end 88.369 103.0639) (width 0.2) (layer "B.Cu") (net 15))
 (segment (start 81.396669 134.65) (end 85.807668 130.239001) (width 0.2) (layer "B.Cu") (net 15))
 (segment (start 95.508 105.914) (end 94.107 107.315) (width 0.2) (layer "B.Cu") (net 15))
 (segment (start 84.620669 116.176) (end 85.456 115.340669) (width 0.2) (layer "B.Cu") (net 15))
 (segment (start 83.9575 123.675) (end 80.0275 123.675) (width 0.2) (layer "B.Cu") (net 15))
 (segment (start 85.807668 130.239001) (end 96.012 130.239001) (width 0.2) (layer "B.Cu") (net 15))
 (segment (start 81.024 116.176) (end 84.620669 116.176) (width 0.2) (layer "B.Cu") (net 15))
 (segment (start 88.369 98.568001) (end 91.183001 95.754) (width 0.2) (layer "B.Cu") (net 15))
 (segment (start 80.1 114.75) (end 79.17 113.82) (width 0.2) (layer "B.Cu") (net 15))
 (segment (start 79.0975 122.745) (end 79.0975 118.1025) (width 0.2) (layer "B.Cu") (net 15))
 (segment (start 91.183001 95.754) (end 94.687314 95.754) (width 0.2) (layer "B.Cu") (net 15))
 (segment (start 85.456 114.159331) (end 84.620669 113.324) (width 0.2) (layer "B.Cu") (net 15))
 (segment (start 80.0275 123.675) (end 79.0975 122.745) (width 0.2) (layer "B.Cu") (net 15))
 (segment (start 95.508 96.574686) (end 95.508 105.914) (width 0.2) (layer "B.Cu") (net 15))
 (segment (start 85.456 115.340669) (end 85.456 114.159331) (width 0.2) (layer "B.Cu") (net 15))
 (segment (start 86.402002 103.081998) (end 90.17 99.314) (width 1.5) (layer "F.Cu") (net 19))
 (segment (start 85.298998 103.081998) (end 86.402002 103.081998) (width 0.2) (layer "F.Cu") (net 19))
 (segment (start 64.872 80.326) (end 64.389 79.843) (width 2) (layer "B.Cu") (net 22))
 (segment (start 74.139 78.526) (end 72.339 80.326) (width 4) (layer "B.Cu") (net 22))
 (segment (start 72.339 80.326) (end 64.872 80.326) (width 4) (layer "B.Cu") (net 22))
 (segment (start 74.139 68.326) (end 74.139 78.526) (width 4) (layer "B.Cu") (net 22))
 (segment (start 94.456 74.843) (end 64.389 74.843) (width 4) (layer "F.Cu") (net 23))
 (segment (start 99.939 80.326) (end 94.456 74.843) (width 4) (layer "F.Cu") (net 23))
 (segment (start 73.675768 137.838) (end 90.412999 137.838) (width 0.2) (layer "F.Cu") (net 20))
 (segment (start 76.594 90.297) (end 72.898 90.297) (width 0.5) (layer "F.Cu") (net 20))
 (segment (start 73.675768 137.838) (end 89.772626 137.838) (width 0.2) (layer "F.Cu") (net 20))
 (segment (start 74.162 98.389) (end 72.344 98.389) (width 0.2) (layer "F.Cu") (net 20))
 (segment (start 70.745 134.907232) (end 73.675768 137.838) (width 0.2) (layer "F.Cu") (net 20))
 (segment (start 71.6975 121.3) (end 73.5985 119.399) (width 0.2) (layer "F.Cu") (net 20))
 (segment (start 73.5985 119.399) (end 73.5985 110.469499) (width 0.2) (layer "F.Cu") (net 20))
 (segment (start 72.898 90.297) (end 70.485 87.884) (width 0.5) (layer "F.Cu") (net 20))
 (segment (start 89.772626 137.838) (end 96.9734 130.637226) (width 0.2) (layer "F.Cu") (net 20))
 (segment (start 71.87 121.4725) (end 71.6975 121.3) (width 0.2) (layer "F.Cu") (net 20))
 (segment (start 71.755 108.625999) (end 71.755 97.8) (width 0.5) (layer "F.Cu") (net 20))
 (segment (start 71.87 132.275) (end 70.745 133.4) (width 0.2) (layer "F.Cu") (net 20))
 (segment (start 76.594 91.457) (end 74.162 93.889) (width 0.5) (layer "F.Cu") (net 20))
 (segment (start 96.9734 129.200399) (end 96.012 128.238999) (width 0.2) (layer "F.Cu") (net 20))
 (segment (start 71.755 96.296) (end 74.162 93.889) (width 0.5) (layer "F.Cu") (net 20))
 (segment (start 76.594 90.297) (end 76.594 91.457) (width 0.5) (layer "F.Cu") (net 20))
 (segment (start 70.745 133.4) (end 70.745 134.907232) (width 0.2) (layer "F.Cu") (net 20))
 (segment (start 90.412999 137.838) (end 96.012 132.238999) (width 0.2) (layer "F.Cu") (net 20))
 (segment (start 76.594 90.297) (end 76.594 90.056) (width 0.5) (layer "F.Cu") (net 20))
 (segment (start 71.87 132.275) (end 71.87 121.4725) (width 0.2) (layer "F.Cu") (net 20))
 (segment (start 71.755 97.8) (end 71.755 96.296) (width 0.5) (layer "F.Cu") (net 20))
 (segment (start 96.9734 130.637226) (end 96.9734 129.200399) (width 0.2) (layer "F.Cu") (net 20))
 (segment (start 73.5985 110.469499) (end 71.755 108.625999) (width 0.2) (layer "F.Cu") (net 20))
 (segment (start 72.344 98.389) (end 71.755 97.8) (width 0.2) (layer "F.Cu") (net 20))
 (segment (start 84.03 114.75) (end 86.242 112.538) (width 1.5) (layer "F.Cu") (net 25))
 (segment (start 86.242 112.538) (end 87.9 112.538) (width 1.5) (layer "F.Cu") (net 25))
 (segment (start 87.9 112.538) (end 95.601 120.239) (width 1.5) (layer "F.Cu") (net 25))
 (segment (start 95.601 120.239) (end 96.012 120.239) (width 1.5) (layer "F.Cu") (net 25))
 (segment (start 84.03 114.75) (end 83.1 115.68) (width 0.2) (layer "B.Cu") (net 25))
 (segment (start 72.982998 103.081998) (end 68.667 98.766) (width 3.5) (layer "B.Cu") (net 25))
 (segment (start 78.769 103.612998) (end 79.3 103.081998) (width 0.2) (layer "B.Cu") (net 25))
 (segment (start 78.769 114.734219) (end 78.769 103.612998) (width 0.2) (layer "B.Cu") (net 25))
 (segment (start 79.3 103.081998) (end 72.982998 103.081998) (width 3.5) (layer "B.Cu") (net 25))
 (segment (start 83.1 115.68) (end 79.714781 115.68) (width 0.2) (layer "B.Cu") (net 25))
 (segment (start 79.714781 115.68) (end 78.769 114.734219) (width 0.2) (layer "B.Cu") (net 25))
 (segment (start 68.667 98.766) (end 68.667 95.377) (width 3.5) (layer "B.Cu") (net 25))
 (segment (start 97.663 93.472) (end 99.441 95.25) (width 0.5) (layer "F.Cu") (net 18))
 (segment (start 99.441 95.25) (end 99.441 122.810001) (width 0.5) (layer "F.Cu") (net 18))
 (segment (start 99.441 122.810001) (end 96.012 126.239001) (width 0.5) (layer "F.Cu") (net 18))
 (segment (start 95.375999 126.239001) (end 96.012 126.239001) (width 0.5) (layer "F.Cu") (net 18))
 (segment (start 84.13 129.9) (end 87.790999 126.239001) (width 0.2) (layer "B.Cu") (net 18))
 (segment (start 87.790999 126.239001) (end 96.012 126.239001) (width 0.2) (layer "B.Cu") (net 18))
 (segment (start 97.663 134.239) (end 96.012 134.239) (width 2) (layer "B.Cu") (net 24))
 (segment (start 99.441 85.344) (end 99.441 132.461) (width 2) (layer "B.Cu") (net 24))
 (segment (start 96.139 82.042) (end 99.441 85.344) (width 2) (layer "B.Cu") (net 24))
 (segment (start 99.441 132.461) (end 97.663 134.239) (width 2) (layer "B.Cu") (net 24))
 (segment (start 96.139 68.326) (end 96.139 82.042) (width 2) (layer "B.Cu") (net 24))
 (segment (start 90.885 101.115) (end 90.915999 101.115) (width 0.2) (layer "B.Cu") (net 16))
 (segment (start 73.417 136.683) (end 63.810108 136.683) (width 0.2) (layer "B.Cu") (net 16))
 (segment (start 67.817448 93.326) (end 69.516552 93.326) (width 0.2) (layer "B.Cu") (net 16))
 (segment (start 63.048 135.920892) (end 63.048 98.095448) (width 0.2) (layer "B.Cu") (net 16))
 (segment (start 81.4535 117.499) (end 84.701 117.499) (width 0.2) (layer "B.Cu") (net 16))
 (segment (start 94.853414 95.353) (end 95.909 96.408586) (width 0.2) (layer "B.Cu") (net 16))
 (segment (start 80.1 110) (end 82 110) (width 0.2) (layer "B.Cu") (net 16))
 (segment (start 69.516552 93.326) (end 71.543552 95.353) (width 0.2) (layer "B.Cu") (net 16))
 (segment (start 90.915999 101.115) (end 91.615499 100.415499) (width 0.2) (layer "B.Cu") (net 16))
 (segment (start 82 110) (end 87.1 115.1) (width 0.2) (layer "B.Cu") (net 16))
 (segment (start 95.909 108.315) (end 95.508 108.716) (width 0.2) (layer "B.Cu") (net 16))
 (segment (start 92.706 108.716) (end 91.615499 107.625499) (width 0.2) (layer "B.Cu") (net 16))
 (segment (start 63.048 98.095448) (end 67.817448 93.326) (width 0.2) (layer "B.Cu") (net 16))
 (segment (start 71.543552 95.353) (end 94.853414 95.353) (width 0.2) (layer "B.Cu") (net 16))
 (segment (start 95.909 96.408586) (end 95.909 108.315) (width 0.2) (layer "B.Cu") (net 16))
 (segment (start 84.701 117.499) (end 87.1 115.1) (width 0.2) (layer "B.Cu") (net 16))
 (segment (start 95.508 108.716) (end 92.706 108.716) (width 0.2) (layer "B.Cu") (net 16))
 (segment (start 80.0275 118.925) (end 81.4535 117.499) (width 0.2) (layer "B.Cu") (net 16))
 (segment (start 63.810108 136.683) (end 63.048 135.920892) (width 0.2) (layer "B.Cu") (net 16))
 (segment (start 80.2 129.9) (end 73.417 136.683) (width 0.2) (layer "B.Cu") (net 16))
 (segment (start 94.107 97.923999) (end 94.107 97.155) (width 0.2) (layer "B.Cu") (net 16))
 (segment (start 82 110) (end 90.885 101.115) (width 0.2) (layer "B.Cu") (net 16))
 (segment (start 87.1 115.1) (end 95.6 123.6) (width 0.2) (layer "B.Cu") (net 16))
 (segment (start 91.615499 100.415499) (end 94.107 97.923999) (width 0.2) (layer "B.Cu") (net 16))
 (segment (start 91.615499 107.625499) (end 91.615499 100.415499) (width 0.2) (layer "B.Cu") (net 16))
 (segment (start 66.298999 98.008999) (end 66.298999 107.001499) (width 3) (layer "F.Cu") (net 30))
 (segment (start 66.298999 107.001499) (end 71.7975 112.5) (width 3) (layer "F.Cu") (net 30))
 (segment (start 63.667 95.377) (end 66.298999 98.008999) (width 3) (layer "F.Cu") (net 30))
 (segment (start 94.615 90.297) (end 94.615 93.472) (width 0.5) (layer "F.Cu") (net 17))
 (segment (start 94.742 90.424) (end 94.615 90.297) (width 0.2) (layer "F.Cu") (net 17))
 (segment (start 94.615 90.297) (end 94.615 87.63) (width 0.5) (layer "F.Cu") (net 17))
 (segment (start 94.615 87.63) (end 94.742 87.503) (width 0.2) (layer "F.Cu") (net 17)))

